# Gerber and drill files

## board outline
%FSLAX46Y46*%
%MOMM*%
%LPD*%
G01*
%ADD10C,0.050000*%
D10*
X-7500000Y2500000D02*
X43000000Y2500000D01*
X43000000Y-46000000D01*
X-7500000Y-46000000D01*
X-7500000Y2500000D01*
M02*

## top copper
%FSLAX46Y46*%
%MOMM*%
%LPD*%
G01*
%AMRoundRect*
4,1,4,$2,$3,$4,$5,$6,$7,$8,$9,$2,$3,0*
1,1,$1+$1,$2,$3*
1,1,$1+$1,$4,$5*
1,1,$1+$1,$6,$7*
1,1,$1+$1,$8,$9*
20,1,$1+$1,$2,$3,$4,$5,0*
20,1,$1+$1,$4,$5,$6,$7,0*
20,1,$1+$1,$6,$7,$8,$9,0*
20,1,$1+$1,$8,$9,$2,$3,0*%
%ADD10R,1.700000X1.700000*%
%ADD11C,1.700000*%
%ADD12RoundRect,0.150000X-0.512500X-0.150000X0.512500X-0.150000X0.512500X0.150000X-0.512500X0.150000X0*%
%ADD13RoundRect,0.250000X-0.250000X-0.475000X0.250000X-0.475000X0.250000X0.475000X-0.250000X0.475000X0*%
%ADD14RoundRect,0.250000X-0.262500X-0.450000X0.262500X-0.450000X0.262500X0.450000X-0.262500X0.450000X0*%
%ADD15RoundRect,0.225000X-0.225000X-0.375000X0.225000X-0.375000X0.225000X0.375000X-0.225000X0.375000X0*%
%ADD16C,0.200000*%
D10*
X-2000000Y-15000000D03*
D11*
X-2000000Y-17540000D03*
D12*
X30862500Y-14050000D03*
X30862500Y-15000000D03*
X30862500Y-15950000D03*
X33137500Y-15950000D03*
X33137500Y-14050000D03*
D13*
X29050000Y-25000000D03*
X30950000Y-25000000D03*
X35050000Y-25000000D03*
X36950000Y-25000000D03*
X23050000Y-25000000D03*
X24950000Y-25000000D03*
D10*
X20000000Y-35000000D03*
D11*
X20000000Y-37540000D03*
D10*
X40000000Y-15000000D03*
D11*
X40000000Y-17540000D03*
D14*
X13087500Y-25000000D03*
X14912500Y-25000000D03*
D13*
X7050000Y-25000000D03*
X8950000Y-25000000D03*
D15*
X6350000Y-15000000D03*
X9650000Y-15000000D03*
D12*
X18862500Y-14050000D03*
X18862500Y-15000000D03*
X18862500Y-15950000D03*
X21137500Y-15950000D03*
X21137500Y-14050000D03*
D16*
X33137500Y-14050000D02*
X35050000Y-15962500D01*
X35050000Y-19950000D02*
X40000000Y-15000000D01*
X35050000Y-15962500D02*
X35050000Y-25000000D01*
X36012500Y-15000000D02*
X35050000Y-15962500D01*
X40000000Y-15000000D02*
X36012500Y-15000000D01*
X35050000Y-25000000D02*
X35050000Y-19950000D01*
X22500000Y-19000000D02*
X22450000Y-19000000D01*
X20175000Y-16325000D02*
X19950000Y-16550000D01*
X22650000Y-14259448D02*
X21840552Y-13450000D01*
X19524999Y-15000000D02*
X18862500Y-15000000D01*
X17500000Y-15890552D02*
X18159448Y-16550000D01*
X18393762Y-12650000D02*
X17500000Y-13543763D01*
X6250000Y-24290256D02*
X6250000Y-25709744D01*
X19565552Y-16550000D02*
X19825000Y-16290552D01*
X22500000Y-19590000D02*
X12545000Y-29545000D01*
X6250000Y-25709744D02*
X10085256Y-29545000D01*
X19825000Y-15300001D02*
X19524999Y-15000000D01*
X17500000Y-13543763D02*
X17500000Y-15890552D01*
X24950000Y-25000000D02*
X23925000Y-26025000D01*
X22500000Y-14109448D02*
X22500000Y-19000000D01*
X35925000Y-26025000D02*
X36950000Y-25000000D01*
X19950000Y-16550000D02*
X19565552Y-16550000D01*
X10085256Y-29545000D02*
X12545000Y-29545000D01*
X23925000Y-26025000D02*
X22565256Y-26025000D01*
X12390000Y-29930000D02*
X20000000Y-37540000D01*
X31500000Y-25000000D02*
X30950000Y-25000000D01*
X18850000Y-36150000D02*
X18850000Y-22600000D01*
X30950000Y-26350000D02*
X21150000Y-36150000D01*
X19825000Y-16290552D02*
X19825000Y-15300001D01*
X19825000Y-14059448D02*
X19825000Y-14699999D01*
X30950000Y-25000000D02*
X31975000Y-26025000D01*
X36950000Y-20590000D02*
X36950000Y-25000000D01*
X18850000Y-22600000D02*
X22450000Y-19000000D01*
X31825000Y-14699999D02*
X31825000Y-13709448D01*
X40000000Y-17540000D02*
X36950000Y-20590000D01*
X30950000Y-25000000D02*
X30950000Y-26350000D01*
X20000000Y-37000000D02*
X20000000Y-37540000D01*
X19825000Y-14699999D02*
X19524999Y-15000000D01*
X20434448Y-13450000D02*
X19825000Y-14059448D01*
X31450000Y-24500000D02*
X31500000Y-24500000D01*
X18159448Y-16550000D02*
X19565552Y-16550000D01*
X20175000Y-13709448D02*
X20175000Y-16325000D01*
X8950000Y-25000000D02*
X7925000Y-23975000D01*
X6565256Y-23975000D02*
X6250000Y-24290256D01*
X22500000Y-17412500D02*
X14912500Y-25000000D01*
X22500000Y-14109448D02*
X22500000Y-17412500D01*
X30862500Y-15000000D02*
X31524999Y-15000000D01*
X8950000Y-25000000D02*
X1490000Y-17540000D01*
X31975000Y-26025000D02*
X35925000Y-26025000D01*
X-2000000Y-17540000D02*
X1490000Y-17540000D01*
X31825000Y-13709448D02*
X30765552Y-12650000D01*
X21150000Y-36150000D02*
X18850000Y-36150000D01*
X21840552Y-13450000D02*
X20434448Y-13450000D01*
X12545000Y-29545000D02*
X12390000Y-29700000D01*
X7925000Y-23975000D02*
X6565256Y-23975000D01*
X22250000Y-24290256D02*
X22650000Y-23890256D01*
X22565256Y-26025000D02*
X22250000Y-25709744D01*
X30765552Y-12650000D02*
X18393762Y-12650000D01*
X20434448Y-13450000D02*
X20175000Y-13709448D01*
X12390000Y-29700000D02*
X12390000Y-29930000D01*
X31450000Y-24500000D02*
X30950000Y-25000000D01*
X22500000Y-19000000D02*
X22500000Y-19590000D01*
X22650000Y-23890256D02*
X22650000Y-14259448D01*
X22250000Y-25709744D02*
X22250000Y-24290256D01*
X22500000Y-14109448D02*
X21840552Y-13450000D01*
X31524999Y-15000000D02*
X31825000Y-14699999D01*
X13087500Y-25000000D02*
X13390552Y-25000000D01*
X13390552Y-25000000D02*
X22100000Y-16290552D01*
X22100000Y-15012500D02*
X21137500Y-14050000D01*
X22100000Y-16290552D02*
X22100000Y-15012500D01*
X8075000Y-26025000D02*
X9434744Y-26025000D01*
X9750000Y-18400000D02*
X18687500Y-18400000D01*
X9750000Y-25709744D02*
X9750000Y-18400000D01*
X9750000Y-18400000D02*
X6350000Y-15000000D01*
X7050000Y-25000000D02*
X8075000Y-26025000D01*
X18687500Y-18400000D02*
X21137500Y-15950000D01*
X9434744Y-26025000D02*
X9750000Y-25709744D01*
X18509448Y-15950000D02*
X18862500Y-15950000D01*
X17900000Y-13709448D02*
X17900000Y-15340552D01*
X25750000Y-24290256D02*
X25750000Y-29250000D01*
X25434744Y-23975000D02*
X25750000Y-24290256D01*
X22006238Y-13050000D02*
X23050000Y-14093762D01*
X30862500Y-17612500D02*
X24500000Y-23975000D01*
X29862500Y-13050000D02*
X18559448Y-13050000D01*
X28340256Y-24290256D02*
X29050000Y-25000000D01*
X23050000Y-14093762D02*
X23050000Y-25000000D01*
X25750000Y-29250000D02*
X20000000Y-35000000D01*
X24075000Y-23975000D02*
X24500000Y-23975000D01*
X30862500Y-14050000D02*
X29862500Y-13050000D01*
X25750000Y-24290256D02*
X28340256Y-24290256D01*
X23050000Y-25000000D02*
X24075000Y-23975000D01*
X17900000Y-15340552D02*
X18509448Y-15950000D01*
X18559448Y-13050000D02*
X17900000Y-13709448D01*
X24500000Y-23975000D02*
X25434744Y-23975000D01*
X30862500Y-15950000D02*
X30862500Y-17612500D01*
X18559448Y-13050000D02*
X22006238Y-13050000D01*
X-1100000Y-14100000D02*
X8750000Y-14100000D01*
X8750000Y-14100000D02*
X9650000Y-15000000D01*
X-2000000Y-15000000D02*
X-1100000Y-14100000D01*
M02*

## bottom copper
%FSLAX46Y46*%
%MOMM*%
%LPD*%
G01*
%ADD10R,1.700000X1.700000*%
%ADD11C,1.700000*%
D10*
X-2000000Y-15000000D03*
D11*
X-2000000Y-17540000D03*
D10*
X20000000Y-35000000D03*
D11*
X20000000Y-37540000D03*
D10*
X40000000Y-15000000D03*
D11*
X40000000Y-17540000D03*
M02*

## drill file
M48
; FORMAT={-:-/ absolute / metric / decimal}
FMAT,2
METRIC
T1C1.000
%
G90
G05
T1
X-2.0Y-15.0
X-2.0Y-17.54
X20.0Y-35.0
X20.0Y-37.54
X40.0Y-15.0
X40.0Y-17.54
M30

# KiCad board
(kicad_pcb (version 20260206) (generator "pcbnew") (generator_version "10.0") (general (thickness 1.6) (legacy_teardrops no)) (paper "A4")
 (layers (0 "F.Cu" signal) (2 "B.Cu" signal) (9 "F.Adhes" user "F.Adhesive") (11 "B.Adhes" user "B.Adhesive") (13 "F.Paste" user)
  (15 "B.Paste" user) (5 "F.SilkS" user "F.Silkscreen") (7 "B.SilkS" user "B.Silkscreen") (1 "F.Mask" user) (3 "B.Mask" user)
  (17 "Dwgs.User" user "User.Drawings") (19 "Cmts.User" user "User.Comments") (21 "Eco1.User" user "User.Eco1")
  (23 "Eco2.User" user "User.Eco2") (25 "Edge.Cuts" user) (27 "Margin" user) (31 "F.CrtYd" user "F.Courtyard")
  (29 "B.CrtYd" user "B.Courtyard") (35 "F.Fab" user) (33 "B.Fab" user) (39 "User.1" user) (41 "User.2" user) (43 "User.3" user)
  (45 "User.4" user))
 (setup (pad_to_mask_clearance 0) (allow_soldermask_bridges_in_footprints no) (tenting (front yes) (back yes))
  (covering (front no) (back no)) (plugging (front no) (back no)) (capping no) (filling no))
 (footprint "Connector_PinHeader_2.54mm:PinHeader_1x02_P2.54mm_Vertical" (layer "F.Cu") (at -2 15)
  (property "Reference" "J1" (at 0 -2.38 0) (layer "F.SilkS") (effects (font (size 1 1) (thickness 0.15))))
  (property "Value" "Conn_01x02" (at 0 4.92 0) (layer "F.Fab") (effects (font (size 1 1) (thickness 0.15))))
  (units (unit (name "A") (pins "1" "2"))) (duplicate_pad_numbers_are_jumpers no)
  (pad "1" thru_hole rect (at 0 0) (size 1.7 1.7) (drill 1) (layers "*.Cu" "*.Mask") (remove_unused_layers no) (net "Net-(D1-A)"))
  (pad "2" thru_hole circle (at 0 2.54) (size 1.7 1.7) (drill 1) (layers "*.Cu" "*.Mask") (remove_unused_layers no) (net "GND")))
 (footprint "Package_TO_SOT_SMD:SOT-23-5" (layer "F.Cu") (at 32 15)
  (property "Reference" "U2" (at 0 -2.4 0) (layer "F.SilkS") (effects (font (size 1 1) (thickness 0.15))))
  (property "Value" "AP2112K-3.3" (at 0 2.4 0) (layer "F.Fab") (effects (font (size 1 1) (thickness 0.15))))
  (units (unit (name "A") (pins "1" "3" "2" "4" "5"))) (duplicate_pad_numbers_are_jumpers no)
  (pad "1" smd roundrect (at -1.1375 -0.95) (size 1.325 0.6) (layers "F.Cu" "F.Mask" "F.Paste") (roundrect_rratio 0.25) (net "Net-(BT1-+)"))
  (pad "2" smd roundrect (at -1.1375 0) (size 1.325 0.6) (layers "F.Cu" "F.Mask" "F.Paste") (roundrect_rratio 0.25) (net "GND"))
  (pad "3" smd roundrect (at -1.1375 0.95) (size 1.325 0.6) (layers "F.Cu" "F.Mask" "F.Paste") (roundrect_rratio 0.25) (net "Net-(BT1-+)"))
  (pad "4" smd roundrect (at 1.1375 0.95) (size 1.325 0.6) (layers "F.Cu" "F.Mask" "F.Paste") (roundrect_rratio 0.25)
   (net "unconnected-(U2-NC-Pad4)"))
  (pad "5" smd roundrect (at 1.1375 -0.95) (size 1.325 0.6) (layers "F.Cu" "F.Mask" "F.Paste") (roundrect_rratio 0.25)
   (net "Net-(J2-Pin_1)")))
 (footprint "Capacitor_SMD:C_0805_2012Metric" (layer "F.Cu") (at 30 25)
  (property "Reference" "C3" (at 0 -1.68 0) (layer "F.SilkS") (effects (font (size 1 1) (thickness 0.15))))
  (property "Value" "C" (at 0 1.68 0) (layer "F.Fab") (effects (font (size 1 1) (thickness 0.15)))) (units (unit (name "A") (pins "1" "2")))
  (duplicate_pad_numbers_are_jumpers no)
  (pad "1" smd roundrect (at -0.95 0) (size 1 1.45) (layers "F.Cu" "F.Mask" "F.Paste") (roundrect_rratio 0.25) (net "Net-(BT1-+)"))
  (pad "2" smd roundrect (at 0.95 0) (size 1 1.45) (layers "F.Cu" "F.Mask" "F.Paste") (roundrect_rratio 0.25) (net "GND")))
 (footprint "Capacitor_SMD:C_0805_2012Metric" (layer "F.Cu") (at 36 25)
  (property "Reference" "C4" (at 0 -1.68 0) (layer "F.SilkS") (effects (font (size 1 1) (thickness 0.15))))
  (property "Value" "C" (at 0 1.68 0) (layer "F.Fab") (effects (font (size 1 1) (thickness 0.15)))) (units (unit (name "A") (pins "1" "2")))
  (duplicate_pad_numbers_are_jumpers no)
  (pad "1" smd roundrect (at -0.95 0) (size 1 1.45) (layers "F.Cu" "F.Mask" "F.Paste") (roundrect_rratio 0.25) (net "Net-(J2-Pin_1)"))
  (pad "2" smd roundrect (at 0.95 0) (size 1 1.45) (layers "F.Cu" "F.Mask" "F.Paste") (roundrect_rratio 0.25) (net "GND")))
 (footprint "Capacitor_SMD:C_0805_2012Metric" (layer "F.Cu") (at 24 25)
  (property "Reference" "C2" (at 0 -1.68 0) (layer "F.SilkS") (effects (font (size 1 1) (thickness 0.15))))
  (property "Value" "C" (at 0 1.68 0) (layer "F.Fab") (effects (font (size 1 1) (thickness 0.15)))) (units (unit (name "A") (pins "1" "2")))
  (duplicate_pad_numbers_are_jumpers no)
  (pad "1" smd roundrect (at -0.95 0) (size 1 1.45) (layers "F.Cu" "F.Mask" "F.Paste") (roundrect_rratio 0.25) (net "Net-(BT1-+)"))
  (pad "2" smd roundrect (at 0.95 0) (size 1 1.45) (layers "F.Cu" "F.Mask" "F.Paste") (roundrect_rratio 0.25) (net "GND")))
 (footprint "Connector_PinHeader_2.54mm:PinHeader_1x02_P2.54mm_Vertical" (layer "F.Cu") (at 20 35)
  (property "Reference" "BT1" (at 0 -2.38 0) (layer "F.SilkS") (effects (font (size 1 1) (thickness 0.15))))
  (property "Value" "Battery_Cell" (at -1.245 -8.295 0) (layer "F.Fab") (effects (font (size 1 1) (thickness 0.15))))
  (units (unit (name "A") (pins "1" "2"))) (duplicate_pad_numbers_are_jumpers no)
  (pad "1" thru_hole rect (at 0 0) (size 1.7 1.7) (drill 1) (layers "*.Cu" "*.Mask") (remove_unused_layers no) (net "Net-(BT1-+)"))
  (pad "2" thru_hole circle (at 0 2.54) (size 1.7 1.7) (drill 1) (layers "*.Cu" "*.Mask") (remove_unused_layers no) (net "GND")))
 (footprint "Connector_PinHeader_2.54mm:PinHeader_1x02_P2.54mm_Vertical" (layer "F.Cu") (at 40 15)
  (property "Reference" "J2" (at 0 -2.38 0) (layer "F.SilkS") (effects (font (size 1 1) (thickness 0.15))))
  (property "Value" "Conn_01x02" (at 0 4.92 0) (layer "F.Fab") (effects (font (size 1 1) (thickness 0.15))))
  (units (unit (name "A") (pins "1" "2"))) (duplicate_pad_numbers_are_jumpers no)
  (pad "1" thru_hole rect (at 0 0) (size 1.7 1.7) (drill 1) (layers "*.Cu" "*.Mask") (remove_unused_layers no) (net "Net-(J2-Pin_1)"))
  (pad "2" thru_hole circle (at 0 2.54) (size 1.7 1.7) (drill 1) (layers "*.Cu" "*.Mask") (remove_unused_layers no) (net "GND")))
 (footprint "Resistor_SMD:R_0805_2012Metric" (layer "F.Cu") (at 14 25)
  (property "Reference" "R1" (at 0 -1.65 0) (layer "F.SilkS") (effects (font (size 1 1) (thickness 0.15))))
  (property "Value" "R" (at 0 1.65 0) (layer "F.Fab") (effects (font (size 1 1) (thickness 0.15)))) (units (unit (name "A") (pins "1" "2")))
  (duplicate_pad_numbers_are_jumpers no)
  (pad "1" smd roundrect (at -0.9125 0) (size 1.025 1.4) (layers "F.Cu" "F.Mask" "F.Paste") (roundrect_rratio 0.243902)
   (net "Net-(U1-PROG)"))
  (pad "2" smd roundrect (at 0.9125 0) (size 1.025 1.4) (layers "F.Cu" "F.Mask" "F.Paste") (roundrect_rratio 0.243902) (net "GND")))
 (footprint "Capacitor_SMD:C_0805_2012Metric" (layer "F.Cu") (at 8 25)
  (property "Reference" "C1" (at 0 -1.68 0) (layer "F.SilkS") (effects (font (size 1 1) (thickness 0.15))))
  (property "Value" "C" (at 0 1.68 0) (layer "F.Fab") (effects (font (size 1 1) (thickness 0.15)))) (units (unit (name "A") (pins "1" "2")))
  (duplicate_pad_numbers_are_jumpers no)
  (pad "1" smd roundrect (at -0.95 0) (size 1 1.45) (layers "F.Cu" "F.Mask" "F.Paste") (roundrect_rratio 0.25) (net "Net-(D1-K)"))
  (pad "2" smd roundrect (at 0.95 0) (size 1 1.45) (layers "F.Cu" "F.Mask" "F.Paste") (roundrect_rratio 0.25) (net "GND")))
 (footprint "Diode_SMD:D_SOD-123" (layer "F.Cu") (at 8 15)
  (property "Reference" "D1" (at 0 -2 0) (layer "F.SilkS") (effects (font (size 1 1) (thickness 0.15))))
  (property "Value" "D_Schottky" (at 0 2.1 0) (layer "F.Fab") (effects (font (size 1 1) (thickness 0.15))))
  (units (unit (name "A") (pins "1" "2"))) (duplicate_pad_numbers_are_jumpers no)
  (pad "1" smd roundrect (at -1.65 0) (size 0.9 1.2) (layers "F.Cu" "F.Mask" "F.Paste") (roundrect_rratio 0.25) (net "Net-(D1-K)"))
  (pad "2" smd roundrect (at 1.65 0) (size 0.9 1.2) (layers "F.Cu" "F.Mask" "F.Paste") (roundrect_rratio 0.25) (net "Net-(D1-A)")))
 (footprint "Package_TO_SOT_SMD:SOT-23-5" (layer "F.Cu") (at 20 15)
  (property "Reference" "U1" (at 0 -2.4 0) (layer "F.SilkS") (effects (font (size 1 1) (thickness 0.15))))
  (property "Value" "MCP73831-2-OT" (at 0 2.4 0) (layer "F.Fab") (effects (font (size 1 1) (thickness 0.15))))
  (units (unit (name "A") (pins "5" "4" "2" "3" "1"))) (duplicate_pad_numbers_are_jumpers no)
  (pad "1" smd roundrect (at -1.1375 -0.95) (size 1.325 0.6) (layers "F.Cu" "F.Mask" "F.Paste") (roundrect_rratio 0.25)
   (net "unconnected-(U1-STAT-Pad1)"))
  (pad "2" smd roundrect (at -1.1375 0) (size 1.325 0.6) (layers "F.Cu" "F.Mask" "F.Paste") (roundrect_rratio 0.25) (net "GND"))
  (pad "3" smd roundrect (at -1.1375 0.95) (size 1.325 0.6) (layers "F.Cu" "F.Mask" "F.Paste") (roundrect_rratio 0.25) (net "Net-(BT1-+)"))
  (pad "4" smd roundrect (at 1.1375 0.95) (size 1.325 0.6) (layers "F.Cu" "F.Mask" "F.Paste") (roundrect_rratio 0.25) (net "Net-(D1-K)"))
  (pad "5" smd roundrect (at 1.1375 -0.95) (size 1.325 0.6) (layers "F.Cu" "F.Mask" "F.Paste") (roundrect_rratio 0.25) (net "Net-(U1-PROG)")))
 (gr_rect (start -7.5 -2.5) (end 43 46) (stroke (width 0.05) (type default)) (fill no) (layer "Edge.Cuts"))
 (segment (start 33.1375 14.05) (end 35.05 15.9625) (width 0.2) (layer "F.Cu") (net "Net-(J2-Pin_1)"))
 (segment (start 35.05 19.95) (end 40 15) (width 0.2) (layer "F.Cu") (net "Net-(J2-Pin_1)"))
 (segment (start 35.05 15.9625) (end 35.05 25) (width 0.2) (layer "F.Cu") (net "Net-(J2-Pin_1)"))
 (segment (start 36.0125 15) (end 35.05 15.9625) (width 0.2) (layer "F.Cu") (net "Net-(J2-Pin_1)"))
 (segment (start 40 15) (end 36.0125 15) (width 0.2) (layer "F.Cu") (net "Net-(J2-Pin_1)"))
 (segment (start 35.05 25) (end 35.05 19.95) (width 0.2) (layer "F.Cu") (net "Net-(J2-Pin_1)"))
 (segment (start 22.5 19) (end 22.45 19) (width 0.2) (layer "F.Cu") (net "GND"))
 (segment (start 20.175 16.325) (end 19.95 16.55) (width 0.2) (layer "F.Cu") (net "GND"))
 (segment (start 22.65 14.259448) (end 21.840552 13.45) (width 0.2) (layer "F.Cu") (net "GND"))
 (segment (start 19.524999 15) (end 18.8625 15) (width 0.2) (layer "F.Cu") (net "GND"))
 (segment (start 17.5 15.890552) (end 18.159448 16.55) (width 0.2) (layer "F.Cu") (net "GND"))
 (segment (start 18.393762 12.65) (end 17.5 13.543763) (width 0.2) (layer "F.Cu") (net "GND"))
 (segment (start 6.25 24.290256) (end 6.25 25.709744) (width 0.2) (layer "F.Cu") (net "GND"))
 (segment (start 19.565552 16.55) (end 19.825 16.290552) (width 0.2) (layer "F.Cu") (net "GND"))
 (segment (start 22.5 19.59) (end 12.545 29.545) (width 0.2) (layer "F.Cu") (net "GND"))
 (segment (start 6.25 25.709744) (end 10.085256 29.545) (width 0.2) (layer "F.Cu") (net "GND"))
 (segment (start 19.825 15.300001) (end 19.524999 15) (width 0.2) (layer "F.Cu") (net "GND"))
 (segment (start 17.5 13.543763) (end 17.5 15.890552) (width 0.2) (layer "F.Cu") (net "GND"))
 (segment (start 24.95 25) (end 23.925 26.025) (width 0.2) (layer "F.Cu") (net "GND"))
 (segment (start 22.5 14.109448) (end 22.5 19) (width 0.2) (layer "F.Cu") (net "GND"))
 (segment (start 35.925 26.025) (end 36.95 25) (width 0.2) (layer "F.Cu") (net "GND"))
 (segment (start 19.95 16.55) (end 19.565552 16.55) (width 0.2) (layer "F.Cu") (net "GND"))
 (segment (start 10.085256 29.545) (end 12.545 29.545) (width 0.2) (layer "F.Cu") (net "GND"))
 (segment (start 23.925 26.025) (end 22.565256 26.025) (width 0.2) (layer "F.Cu") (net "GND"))
 (segment (start 12.39 29.93) (end 20 37.54) (width 0.2) (layer "F.Cu") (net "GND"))
 (segment (start 31.5 25) (end 30.95 25) (width 0.2) (layer "F.Cu") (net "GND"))
 (segment (start 18.85 36.15) (end 18.85 22.6) (width 0.2) (layer "F.Cu") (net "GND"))
 (segment (start 30.95 26.35) (end 21.15 36.15) (width 0.2) (layer "F.Cu") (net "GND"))
 (segment (start 19.825 16.290552) (end 19.825 15.300001) (width 0.2) (layer "F.Cu") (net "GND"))
 (segment (start 19.825 14.059448) (end 19.825 14.699999) (width 0.2) (layer "F.Cu") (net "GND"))
 (segment (start 30.95 25) (end 31.975 26.025) (width 0.2) (layer "F.Cu") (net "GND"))
 (segment (start 36.95 20.59) (end 36.95 25) (width 0.2) (layer "F.Cu") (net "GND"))
 (segment (start 18.85 22.6) (end 22.45 19) (width 0.2) (layer "F.Cu") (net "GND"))
 (segment (start 31.825 14.699999) (end 31.825 13.709448) (width 0.2) (layer "F.Cu") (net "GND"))
 (segment (start 40 17.54) (end 36.95 20.59) (width 0.2) (layer "F.Cu") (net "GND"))
 (segment (start 30.95 25) (end 30.95 26.35) (width 0.2) (layer "F.Cu") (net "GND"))
 (segment (start 20 37) (end 20 37.54) (width 0.2) (layer "F.Cu") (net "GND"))
 (segment (start 19.825 14.699999) (end 19.524999 15) (width 0.2) (layer "F.Cu") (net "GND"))
 (segment (start 20.434448 13.45) (end 19.825 14.059448) (width 0.2) (layer "F.Cu") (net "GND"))
 (segment (start 31.45 24.5) (end 31.5 24.5) (width 0.2) (layer "F.Cu") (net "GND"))
 (segment (start 18.159448 16.55) (end 19.565552 16.55) (width 0.2) (layer "F.Cu") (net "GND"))
 (segment (start 20.175 13.709448) (end 20.175 16.325) (width 0.2) (layer "F.Cu") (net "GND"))
 (segment (start 8.95 25) (end 7.925 23.975) (width 0.2) (layer "F.Cu") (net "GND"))
 (segment (start 6.565256 23.975) (end 6.25 24.290256) (width 0.2) (layer "F.Cu") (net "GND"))
 (segment (start 22.5 17.4125) (end 14.9125 25) (width 0.2) (layer "F.Cu") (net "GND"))
 (segment (start 22.5 14.109448) (end 22.5 17.4125) (width 0.2) (layer "F.Cu") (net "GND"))
 (segment (start 30.8625 15) (end 31.524999 15) (width 0.2) (layer "F.Cu") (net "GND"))
 (segment (start 8.95 25) (end 1.49 17.54) (width 0.2) (layer "F.Cu") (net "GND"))
 (segment (start 31.975 26.025) (end 35.925 26.025) (width 0.2) (layer "F.Cu") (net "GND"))
 (segment (start -2 17.54) (end 1.49 17.54) (width 0.2) (layer "F.Cu") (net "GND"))
 (segment (start 31.825 13.709448) (end 30.765552 12.65) (width 0.2) (layer "F.Cu") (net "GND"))
 (segment (start 21.15 36.15) (end 18.85 36.15) (width 0.2) (layer "F.Cu") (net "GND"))
 (segment (start 21.840552 13.45) (end 20.434448 13.45) (width 0.2) (layer "F.Cu") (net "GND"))
 (segment (start 12.545 29.545) (end 12.39 29.7) (width 0.2) (layer "F.Cu") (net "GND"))
 (segment (start 7.925 23.975) (end 6.565256 23.975) (width 0.2) (layer "F.Cu") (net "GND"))
 (segment (start 22.25 24.290256) (end 22.65 23.890256) (width 0.2) (layer "F.Cu") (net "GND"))
 (segment (start 22.565256 26.025) (end 22.25 25.709744) (width 0.2) (layer "F.Cu") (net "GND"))
 (segment (start 30.765552 12.65) (end 18.393762 12.65) (width 0.2) (layer "F.Cu") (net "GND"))
 (segment (start 20.434448 13.45) (end 20.175 13.709448) (width 0.2) (layer "F.Cu") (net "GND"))
 (segment (start 12.39 29.7) (end 12.39 29.93) (width 0.2) (layer "F.Cu") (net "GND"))
 (segment (start 31.45 24.5) (end 30.95 25) (width 0.2) (layer "F.Cu") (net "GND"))
 (segment (start 22.5 19) (end 22.5 19.59) (width 0.2) (layer "F.Cu") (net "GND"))
 (segment (start 22.65 23.890256) (end 22.65 14.259448) (width 0.2) (layer "F.Cu") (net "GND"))
 (segment (start 22.25 25.709744) (end 22.25 24.290256) (width 0.2) (layer "F.Cu") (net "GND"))
 (segment (start 22.5 14.109448) (end 21.840552 13.45) (width 0.2) (layer "F.Cu") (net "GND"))
 (segment (start 31.524999 15) (end 31.825 14.699999) (width 0.2) (layer "F.Cu") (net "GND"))
 (segment (start 13.0875 25) (end 13.390552 25) (width 0.2) (layer "F.Cu") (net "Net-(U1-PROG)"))
 (segment (start 13.390552 25) (end 22.1 16.290552) (width 0.2) (layer "F.Cu") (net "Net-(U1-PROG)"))
 (segment (start 22.1 15.0125) (end 21.1375 14.05) (width 0.2) (layer "F.Cu") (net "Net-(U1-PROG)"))
 (segment (start 22.1 16.290552) (end 22.1 15.0125) (width 0.2) (layer "F.Cu") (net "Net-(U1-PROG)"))
 (segment (start 8.075 26.025) (end 9.434744 26.025) (width 0.2) (layer "F.Cu") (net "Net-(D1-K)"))
 (segment (start 9.75 18.4) (end 18.6875 18.4) (width 0.2) (layer "F.Cu") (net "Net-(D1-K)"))
 (segment (start 9.75 25.709744) (end 9.75 18.4) (width 0.2) (layer "F.Cu") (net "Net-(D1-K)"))
 (segment (start 9.75 18.4) (end 6.35 15) (width 0.2) (layer "F.Cu") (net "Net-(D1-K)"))
 (segment (start 7.05 25) (end 8.075 26.025) (width 0.2) (layer "F.Cu") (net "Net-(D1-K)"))
 (segment (start 18.6875 18.4) (end 21.1375 15.95) (width 0.2) (layer "F.Cu") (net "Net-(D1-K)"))
 (segment (start 9.434744 26.025) (end 9.75 25.709744) (width 0.2) (layer "F.Cu") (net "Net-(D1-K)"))
 (segment (start 18.509448 15.95) (end 18.8625 15.95) (width 0.2) (layer "F.Cu") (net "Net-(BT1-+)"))
 (segment (start 17.9 13.709448) (end 17.9 15.340552) (width 0.2) (layer "F.Cu") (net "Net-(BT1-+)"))
 (segment (start 25.75 24.290256) (end 25.75 29.25) (width 0.2) (layer "F.Cu") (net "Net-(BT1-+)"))
 (segment (start 25.434744 23.975) (end 25.75 24.290256) (width 0.2) (layer "F.Cu") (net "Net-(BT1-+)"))
 (segment (start 22.006238 13.05) (end 23.05 14.093762) (width 0.2) (layer "F.Cu") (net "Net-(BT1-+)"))
 (segment (start 30.8625 17.6125) (end 24.5 23.975) (width 0.2) (layer "F.Cu") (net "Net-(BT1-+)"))
 (segment (start 29.8625 13.05) (end 18.559448 13.05) (width 0.2) (layer "F.Cu") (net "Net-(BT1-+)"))
 (segment (start 28.340256 24.290256) (end 29.05 25) (width 0.2) (layer "F.Cu") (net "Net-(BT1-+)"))
 (segment (start 23.05 14.093762) (end 23.05 25) (width 0.2) (layer "F.Cu") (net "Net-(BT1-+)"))
 (segment (start 25.75 29.25) (end 20 35) (width 0.2) (layer "F.Cu") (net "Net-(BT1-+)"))
 (segment (start 24.075 23.975) (end 24.5 23.975) (width 0.2) (layer "F.Cu") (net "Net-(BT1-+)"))
 (segment (start 30.8625 14.05) (end 29.8625 13.05) (width 0.2) (layer "F.Cu") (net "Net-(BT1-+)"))
 (segment (start 25.75 24.290256) (end 28.340256 24.290256) (width 0.2) (layer "F.Cu") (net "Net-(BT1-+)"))
 (segment (start 23.05 25) (end 24.075 23.975) (width 0.2) (layer "F.Cu") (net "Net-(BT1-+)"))
 (segment (start 17.9 15.340552) (end 18.509448 15.95) (width 0.2) (layer "F.Cu") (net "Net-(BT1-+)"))
 (segment (start 18.559448 13.05) (end 17.9 13.709448) (width 0.2) (layer "F.Cu") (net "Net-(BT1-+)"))
 (segment (start 24.5 23.975) (end 25.434744 23.975) (width 0.2) (layer "F.Cu") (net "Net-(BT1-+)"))
 (segment (start 30.8625 15.95) (end 30.8625 17.6125) (width 0.2) (layer "F.Cu") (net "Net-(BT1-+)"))
 (segment (start 18.559448 13.05) (end 22.006238 13.05) (width 0.2) (layer "F.Cu") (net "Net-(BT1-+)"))
 (segment (start -1.1 14.1) (end 8.75 14.1) (width 0.2) (layer "F.Cu") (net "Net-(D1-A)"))
 (segment (start 8.75 14.1) (end 9.65 15) (width 0.2) (layer "F.Cu") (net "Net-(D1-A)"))
 (segment (start -2 15) (end -1.1 14.1) (width 0.2) (layer "F.Cu") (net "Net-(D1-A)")))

